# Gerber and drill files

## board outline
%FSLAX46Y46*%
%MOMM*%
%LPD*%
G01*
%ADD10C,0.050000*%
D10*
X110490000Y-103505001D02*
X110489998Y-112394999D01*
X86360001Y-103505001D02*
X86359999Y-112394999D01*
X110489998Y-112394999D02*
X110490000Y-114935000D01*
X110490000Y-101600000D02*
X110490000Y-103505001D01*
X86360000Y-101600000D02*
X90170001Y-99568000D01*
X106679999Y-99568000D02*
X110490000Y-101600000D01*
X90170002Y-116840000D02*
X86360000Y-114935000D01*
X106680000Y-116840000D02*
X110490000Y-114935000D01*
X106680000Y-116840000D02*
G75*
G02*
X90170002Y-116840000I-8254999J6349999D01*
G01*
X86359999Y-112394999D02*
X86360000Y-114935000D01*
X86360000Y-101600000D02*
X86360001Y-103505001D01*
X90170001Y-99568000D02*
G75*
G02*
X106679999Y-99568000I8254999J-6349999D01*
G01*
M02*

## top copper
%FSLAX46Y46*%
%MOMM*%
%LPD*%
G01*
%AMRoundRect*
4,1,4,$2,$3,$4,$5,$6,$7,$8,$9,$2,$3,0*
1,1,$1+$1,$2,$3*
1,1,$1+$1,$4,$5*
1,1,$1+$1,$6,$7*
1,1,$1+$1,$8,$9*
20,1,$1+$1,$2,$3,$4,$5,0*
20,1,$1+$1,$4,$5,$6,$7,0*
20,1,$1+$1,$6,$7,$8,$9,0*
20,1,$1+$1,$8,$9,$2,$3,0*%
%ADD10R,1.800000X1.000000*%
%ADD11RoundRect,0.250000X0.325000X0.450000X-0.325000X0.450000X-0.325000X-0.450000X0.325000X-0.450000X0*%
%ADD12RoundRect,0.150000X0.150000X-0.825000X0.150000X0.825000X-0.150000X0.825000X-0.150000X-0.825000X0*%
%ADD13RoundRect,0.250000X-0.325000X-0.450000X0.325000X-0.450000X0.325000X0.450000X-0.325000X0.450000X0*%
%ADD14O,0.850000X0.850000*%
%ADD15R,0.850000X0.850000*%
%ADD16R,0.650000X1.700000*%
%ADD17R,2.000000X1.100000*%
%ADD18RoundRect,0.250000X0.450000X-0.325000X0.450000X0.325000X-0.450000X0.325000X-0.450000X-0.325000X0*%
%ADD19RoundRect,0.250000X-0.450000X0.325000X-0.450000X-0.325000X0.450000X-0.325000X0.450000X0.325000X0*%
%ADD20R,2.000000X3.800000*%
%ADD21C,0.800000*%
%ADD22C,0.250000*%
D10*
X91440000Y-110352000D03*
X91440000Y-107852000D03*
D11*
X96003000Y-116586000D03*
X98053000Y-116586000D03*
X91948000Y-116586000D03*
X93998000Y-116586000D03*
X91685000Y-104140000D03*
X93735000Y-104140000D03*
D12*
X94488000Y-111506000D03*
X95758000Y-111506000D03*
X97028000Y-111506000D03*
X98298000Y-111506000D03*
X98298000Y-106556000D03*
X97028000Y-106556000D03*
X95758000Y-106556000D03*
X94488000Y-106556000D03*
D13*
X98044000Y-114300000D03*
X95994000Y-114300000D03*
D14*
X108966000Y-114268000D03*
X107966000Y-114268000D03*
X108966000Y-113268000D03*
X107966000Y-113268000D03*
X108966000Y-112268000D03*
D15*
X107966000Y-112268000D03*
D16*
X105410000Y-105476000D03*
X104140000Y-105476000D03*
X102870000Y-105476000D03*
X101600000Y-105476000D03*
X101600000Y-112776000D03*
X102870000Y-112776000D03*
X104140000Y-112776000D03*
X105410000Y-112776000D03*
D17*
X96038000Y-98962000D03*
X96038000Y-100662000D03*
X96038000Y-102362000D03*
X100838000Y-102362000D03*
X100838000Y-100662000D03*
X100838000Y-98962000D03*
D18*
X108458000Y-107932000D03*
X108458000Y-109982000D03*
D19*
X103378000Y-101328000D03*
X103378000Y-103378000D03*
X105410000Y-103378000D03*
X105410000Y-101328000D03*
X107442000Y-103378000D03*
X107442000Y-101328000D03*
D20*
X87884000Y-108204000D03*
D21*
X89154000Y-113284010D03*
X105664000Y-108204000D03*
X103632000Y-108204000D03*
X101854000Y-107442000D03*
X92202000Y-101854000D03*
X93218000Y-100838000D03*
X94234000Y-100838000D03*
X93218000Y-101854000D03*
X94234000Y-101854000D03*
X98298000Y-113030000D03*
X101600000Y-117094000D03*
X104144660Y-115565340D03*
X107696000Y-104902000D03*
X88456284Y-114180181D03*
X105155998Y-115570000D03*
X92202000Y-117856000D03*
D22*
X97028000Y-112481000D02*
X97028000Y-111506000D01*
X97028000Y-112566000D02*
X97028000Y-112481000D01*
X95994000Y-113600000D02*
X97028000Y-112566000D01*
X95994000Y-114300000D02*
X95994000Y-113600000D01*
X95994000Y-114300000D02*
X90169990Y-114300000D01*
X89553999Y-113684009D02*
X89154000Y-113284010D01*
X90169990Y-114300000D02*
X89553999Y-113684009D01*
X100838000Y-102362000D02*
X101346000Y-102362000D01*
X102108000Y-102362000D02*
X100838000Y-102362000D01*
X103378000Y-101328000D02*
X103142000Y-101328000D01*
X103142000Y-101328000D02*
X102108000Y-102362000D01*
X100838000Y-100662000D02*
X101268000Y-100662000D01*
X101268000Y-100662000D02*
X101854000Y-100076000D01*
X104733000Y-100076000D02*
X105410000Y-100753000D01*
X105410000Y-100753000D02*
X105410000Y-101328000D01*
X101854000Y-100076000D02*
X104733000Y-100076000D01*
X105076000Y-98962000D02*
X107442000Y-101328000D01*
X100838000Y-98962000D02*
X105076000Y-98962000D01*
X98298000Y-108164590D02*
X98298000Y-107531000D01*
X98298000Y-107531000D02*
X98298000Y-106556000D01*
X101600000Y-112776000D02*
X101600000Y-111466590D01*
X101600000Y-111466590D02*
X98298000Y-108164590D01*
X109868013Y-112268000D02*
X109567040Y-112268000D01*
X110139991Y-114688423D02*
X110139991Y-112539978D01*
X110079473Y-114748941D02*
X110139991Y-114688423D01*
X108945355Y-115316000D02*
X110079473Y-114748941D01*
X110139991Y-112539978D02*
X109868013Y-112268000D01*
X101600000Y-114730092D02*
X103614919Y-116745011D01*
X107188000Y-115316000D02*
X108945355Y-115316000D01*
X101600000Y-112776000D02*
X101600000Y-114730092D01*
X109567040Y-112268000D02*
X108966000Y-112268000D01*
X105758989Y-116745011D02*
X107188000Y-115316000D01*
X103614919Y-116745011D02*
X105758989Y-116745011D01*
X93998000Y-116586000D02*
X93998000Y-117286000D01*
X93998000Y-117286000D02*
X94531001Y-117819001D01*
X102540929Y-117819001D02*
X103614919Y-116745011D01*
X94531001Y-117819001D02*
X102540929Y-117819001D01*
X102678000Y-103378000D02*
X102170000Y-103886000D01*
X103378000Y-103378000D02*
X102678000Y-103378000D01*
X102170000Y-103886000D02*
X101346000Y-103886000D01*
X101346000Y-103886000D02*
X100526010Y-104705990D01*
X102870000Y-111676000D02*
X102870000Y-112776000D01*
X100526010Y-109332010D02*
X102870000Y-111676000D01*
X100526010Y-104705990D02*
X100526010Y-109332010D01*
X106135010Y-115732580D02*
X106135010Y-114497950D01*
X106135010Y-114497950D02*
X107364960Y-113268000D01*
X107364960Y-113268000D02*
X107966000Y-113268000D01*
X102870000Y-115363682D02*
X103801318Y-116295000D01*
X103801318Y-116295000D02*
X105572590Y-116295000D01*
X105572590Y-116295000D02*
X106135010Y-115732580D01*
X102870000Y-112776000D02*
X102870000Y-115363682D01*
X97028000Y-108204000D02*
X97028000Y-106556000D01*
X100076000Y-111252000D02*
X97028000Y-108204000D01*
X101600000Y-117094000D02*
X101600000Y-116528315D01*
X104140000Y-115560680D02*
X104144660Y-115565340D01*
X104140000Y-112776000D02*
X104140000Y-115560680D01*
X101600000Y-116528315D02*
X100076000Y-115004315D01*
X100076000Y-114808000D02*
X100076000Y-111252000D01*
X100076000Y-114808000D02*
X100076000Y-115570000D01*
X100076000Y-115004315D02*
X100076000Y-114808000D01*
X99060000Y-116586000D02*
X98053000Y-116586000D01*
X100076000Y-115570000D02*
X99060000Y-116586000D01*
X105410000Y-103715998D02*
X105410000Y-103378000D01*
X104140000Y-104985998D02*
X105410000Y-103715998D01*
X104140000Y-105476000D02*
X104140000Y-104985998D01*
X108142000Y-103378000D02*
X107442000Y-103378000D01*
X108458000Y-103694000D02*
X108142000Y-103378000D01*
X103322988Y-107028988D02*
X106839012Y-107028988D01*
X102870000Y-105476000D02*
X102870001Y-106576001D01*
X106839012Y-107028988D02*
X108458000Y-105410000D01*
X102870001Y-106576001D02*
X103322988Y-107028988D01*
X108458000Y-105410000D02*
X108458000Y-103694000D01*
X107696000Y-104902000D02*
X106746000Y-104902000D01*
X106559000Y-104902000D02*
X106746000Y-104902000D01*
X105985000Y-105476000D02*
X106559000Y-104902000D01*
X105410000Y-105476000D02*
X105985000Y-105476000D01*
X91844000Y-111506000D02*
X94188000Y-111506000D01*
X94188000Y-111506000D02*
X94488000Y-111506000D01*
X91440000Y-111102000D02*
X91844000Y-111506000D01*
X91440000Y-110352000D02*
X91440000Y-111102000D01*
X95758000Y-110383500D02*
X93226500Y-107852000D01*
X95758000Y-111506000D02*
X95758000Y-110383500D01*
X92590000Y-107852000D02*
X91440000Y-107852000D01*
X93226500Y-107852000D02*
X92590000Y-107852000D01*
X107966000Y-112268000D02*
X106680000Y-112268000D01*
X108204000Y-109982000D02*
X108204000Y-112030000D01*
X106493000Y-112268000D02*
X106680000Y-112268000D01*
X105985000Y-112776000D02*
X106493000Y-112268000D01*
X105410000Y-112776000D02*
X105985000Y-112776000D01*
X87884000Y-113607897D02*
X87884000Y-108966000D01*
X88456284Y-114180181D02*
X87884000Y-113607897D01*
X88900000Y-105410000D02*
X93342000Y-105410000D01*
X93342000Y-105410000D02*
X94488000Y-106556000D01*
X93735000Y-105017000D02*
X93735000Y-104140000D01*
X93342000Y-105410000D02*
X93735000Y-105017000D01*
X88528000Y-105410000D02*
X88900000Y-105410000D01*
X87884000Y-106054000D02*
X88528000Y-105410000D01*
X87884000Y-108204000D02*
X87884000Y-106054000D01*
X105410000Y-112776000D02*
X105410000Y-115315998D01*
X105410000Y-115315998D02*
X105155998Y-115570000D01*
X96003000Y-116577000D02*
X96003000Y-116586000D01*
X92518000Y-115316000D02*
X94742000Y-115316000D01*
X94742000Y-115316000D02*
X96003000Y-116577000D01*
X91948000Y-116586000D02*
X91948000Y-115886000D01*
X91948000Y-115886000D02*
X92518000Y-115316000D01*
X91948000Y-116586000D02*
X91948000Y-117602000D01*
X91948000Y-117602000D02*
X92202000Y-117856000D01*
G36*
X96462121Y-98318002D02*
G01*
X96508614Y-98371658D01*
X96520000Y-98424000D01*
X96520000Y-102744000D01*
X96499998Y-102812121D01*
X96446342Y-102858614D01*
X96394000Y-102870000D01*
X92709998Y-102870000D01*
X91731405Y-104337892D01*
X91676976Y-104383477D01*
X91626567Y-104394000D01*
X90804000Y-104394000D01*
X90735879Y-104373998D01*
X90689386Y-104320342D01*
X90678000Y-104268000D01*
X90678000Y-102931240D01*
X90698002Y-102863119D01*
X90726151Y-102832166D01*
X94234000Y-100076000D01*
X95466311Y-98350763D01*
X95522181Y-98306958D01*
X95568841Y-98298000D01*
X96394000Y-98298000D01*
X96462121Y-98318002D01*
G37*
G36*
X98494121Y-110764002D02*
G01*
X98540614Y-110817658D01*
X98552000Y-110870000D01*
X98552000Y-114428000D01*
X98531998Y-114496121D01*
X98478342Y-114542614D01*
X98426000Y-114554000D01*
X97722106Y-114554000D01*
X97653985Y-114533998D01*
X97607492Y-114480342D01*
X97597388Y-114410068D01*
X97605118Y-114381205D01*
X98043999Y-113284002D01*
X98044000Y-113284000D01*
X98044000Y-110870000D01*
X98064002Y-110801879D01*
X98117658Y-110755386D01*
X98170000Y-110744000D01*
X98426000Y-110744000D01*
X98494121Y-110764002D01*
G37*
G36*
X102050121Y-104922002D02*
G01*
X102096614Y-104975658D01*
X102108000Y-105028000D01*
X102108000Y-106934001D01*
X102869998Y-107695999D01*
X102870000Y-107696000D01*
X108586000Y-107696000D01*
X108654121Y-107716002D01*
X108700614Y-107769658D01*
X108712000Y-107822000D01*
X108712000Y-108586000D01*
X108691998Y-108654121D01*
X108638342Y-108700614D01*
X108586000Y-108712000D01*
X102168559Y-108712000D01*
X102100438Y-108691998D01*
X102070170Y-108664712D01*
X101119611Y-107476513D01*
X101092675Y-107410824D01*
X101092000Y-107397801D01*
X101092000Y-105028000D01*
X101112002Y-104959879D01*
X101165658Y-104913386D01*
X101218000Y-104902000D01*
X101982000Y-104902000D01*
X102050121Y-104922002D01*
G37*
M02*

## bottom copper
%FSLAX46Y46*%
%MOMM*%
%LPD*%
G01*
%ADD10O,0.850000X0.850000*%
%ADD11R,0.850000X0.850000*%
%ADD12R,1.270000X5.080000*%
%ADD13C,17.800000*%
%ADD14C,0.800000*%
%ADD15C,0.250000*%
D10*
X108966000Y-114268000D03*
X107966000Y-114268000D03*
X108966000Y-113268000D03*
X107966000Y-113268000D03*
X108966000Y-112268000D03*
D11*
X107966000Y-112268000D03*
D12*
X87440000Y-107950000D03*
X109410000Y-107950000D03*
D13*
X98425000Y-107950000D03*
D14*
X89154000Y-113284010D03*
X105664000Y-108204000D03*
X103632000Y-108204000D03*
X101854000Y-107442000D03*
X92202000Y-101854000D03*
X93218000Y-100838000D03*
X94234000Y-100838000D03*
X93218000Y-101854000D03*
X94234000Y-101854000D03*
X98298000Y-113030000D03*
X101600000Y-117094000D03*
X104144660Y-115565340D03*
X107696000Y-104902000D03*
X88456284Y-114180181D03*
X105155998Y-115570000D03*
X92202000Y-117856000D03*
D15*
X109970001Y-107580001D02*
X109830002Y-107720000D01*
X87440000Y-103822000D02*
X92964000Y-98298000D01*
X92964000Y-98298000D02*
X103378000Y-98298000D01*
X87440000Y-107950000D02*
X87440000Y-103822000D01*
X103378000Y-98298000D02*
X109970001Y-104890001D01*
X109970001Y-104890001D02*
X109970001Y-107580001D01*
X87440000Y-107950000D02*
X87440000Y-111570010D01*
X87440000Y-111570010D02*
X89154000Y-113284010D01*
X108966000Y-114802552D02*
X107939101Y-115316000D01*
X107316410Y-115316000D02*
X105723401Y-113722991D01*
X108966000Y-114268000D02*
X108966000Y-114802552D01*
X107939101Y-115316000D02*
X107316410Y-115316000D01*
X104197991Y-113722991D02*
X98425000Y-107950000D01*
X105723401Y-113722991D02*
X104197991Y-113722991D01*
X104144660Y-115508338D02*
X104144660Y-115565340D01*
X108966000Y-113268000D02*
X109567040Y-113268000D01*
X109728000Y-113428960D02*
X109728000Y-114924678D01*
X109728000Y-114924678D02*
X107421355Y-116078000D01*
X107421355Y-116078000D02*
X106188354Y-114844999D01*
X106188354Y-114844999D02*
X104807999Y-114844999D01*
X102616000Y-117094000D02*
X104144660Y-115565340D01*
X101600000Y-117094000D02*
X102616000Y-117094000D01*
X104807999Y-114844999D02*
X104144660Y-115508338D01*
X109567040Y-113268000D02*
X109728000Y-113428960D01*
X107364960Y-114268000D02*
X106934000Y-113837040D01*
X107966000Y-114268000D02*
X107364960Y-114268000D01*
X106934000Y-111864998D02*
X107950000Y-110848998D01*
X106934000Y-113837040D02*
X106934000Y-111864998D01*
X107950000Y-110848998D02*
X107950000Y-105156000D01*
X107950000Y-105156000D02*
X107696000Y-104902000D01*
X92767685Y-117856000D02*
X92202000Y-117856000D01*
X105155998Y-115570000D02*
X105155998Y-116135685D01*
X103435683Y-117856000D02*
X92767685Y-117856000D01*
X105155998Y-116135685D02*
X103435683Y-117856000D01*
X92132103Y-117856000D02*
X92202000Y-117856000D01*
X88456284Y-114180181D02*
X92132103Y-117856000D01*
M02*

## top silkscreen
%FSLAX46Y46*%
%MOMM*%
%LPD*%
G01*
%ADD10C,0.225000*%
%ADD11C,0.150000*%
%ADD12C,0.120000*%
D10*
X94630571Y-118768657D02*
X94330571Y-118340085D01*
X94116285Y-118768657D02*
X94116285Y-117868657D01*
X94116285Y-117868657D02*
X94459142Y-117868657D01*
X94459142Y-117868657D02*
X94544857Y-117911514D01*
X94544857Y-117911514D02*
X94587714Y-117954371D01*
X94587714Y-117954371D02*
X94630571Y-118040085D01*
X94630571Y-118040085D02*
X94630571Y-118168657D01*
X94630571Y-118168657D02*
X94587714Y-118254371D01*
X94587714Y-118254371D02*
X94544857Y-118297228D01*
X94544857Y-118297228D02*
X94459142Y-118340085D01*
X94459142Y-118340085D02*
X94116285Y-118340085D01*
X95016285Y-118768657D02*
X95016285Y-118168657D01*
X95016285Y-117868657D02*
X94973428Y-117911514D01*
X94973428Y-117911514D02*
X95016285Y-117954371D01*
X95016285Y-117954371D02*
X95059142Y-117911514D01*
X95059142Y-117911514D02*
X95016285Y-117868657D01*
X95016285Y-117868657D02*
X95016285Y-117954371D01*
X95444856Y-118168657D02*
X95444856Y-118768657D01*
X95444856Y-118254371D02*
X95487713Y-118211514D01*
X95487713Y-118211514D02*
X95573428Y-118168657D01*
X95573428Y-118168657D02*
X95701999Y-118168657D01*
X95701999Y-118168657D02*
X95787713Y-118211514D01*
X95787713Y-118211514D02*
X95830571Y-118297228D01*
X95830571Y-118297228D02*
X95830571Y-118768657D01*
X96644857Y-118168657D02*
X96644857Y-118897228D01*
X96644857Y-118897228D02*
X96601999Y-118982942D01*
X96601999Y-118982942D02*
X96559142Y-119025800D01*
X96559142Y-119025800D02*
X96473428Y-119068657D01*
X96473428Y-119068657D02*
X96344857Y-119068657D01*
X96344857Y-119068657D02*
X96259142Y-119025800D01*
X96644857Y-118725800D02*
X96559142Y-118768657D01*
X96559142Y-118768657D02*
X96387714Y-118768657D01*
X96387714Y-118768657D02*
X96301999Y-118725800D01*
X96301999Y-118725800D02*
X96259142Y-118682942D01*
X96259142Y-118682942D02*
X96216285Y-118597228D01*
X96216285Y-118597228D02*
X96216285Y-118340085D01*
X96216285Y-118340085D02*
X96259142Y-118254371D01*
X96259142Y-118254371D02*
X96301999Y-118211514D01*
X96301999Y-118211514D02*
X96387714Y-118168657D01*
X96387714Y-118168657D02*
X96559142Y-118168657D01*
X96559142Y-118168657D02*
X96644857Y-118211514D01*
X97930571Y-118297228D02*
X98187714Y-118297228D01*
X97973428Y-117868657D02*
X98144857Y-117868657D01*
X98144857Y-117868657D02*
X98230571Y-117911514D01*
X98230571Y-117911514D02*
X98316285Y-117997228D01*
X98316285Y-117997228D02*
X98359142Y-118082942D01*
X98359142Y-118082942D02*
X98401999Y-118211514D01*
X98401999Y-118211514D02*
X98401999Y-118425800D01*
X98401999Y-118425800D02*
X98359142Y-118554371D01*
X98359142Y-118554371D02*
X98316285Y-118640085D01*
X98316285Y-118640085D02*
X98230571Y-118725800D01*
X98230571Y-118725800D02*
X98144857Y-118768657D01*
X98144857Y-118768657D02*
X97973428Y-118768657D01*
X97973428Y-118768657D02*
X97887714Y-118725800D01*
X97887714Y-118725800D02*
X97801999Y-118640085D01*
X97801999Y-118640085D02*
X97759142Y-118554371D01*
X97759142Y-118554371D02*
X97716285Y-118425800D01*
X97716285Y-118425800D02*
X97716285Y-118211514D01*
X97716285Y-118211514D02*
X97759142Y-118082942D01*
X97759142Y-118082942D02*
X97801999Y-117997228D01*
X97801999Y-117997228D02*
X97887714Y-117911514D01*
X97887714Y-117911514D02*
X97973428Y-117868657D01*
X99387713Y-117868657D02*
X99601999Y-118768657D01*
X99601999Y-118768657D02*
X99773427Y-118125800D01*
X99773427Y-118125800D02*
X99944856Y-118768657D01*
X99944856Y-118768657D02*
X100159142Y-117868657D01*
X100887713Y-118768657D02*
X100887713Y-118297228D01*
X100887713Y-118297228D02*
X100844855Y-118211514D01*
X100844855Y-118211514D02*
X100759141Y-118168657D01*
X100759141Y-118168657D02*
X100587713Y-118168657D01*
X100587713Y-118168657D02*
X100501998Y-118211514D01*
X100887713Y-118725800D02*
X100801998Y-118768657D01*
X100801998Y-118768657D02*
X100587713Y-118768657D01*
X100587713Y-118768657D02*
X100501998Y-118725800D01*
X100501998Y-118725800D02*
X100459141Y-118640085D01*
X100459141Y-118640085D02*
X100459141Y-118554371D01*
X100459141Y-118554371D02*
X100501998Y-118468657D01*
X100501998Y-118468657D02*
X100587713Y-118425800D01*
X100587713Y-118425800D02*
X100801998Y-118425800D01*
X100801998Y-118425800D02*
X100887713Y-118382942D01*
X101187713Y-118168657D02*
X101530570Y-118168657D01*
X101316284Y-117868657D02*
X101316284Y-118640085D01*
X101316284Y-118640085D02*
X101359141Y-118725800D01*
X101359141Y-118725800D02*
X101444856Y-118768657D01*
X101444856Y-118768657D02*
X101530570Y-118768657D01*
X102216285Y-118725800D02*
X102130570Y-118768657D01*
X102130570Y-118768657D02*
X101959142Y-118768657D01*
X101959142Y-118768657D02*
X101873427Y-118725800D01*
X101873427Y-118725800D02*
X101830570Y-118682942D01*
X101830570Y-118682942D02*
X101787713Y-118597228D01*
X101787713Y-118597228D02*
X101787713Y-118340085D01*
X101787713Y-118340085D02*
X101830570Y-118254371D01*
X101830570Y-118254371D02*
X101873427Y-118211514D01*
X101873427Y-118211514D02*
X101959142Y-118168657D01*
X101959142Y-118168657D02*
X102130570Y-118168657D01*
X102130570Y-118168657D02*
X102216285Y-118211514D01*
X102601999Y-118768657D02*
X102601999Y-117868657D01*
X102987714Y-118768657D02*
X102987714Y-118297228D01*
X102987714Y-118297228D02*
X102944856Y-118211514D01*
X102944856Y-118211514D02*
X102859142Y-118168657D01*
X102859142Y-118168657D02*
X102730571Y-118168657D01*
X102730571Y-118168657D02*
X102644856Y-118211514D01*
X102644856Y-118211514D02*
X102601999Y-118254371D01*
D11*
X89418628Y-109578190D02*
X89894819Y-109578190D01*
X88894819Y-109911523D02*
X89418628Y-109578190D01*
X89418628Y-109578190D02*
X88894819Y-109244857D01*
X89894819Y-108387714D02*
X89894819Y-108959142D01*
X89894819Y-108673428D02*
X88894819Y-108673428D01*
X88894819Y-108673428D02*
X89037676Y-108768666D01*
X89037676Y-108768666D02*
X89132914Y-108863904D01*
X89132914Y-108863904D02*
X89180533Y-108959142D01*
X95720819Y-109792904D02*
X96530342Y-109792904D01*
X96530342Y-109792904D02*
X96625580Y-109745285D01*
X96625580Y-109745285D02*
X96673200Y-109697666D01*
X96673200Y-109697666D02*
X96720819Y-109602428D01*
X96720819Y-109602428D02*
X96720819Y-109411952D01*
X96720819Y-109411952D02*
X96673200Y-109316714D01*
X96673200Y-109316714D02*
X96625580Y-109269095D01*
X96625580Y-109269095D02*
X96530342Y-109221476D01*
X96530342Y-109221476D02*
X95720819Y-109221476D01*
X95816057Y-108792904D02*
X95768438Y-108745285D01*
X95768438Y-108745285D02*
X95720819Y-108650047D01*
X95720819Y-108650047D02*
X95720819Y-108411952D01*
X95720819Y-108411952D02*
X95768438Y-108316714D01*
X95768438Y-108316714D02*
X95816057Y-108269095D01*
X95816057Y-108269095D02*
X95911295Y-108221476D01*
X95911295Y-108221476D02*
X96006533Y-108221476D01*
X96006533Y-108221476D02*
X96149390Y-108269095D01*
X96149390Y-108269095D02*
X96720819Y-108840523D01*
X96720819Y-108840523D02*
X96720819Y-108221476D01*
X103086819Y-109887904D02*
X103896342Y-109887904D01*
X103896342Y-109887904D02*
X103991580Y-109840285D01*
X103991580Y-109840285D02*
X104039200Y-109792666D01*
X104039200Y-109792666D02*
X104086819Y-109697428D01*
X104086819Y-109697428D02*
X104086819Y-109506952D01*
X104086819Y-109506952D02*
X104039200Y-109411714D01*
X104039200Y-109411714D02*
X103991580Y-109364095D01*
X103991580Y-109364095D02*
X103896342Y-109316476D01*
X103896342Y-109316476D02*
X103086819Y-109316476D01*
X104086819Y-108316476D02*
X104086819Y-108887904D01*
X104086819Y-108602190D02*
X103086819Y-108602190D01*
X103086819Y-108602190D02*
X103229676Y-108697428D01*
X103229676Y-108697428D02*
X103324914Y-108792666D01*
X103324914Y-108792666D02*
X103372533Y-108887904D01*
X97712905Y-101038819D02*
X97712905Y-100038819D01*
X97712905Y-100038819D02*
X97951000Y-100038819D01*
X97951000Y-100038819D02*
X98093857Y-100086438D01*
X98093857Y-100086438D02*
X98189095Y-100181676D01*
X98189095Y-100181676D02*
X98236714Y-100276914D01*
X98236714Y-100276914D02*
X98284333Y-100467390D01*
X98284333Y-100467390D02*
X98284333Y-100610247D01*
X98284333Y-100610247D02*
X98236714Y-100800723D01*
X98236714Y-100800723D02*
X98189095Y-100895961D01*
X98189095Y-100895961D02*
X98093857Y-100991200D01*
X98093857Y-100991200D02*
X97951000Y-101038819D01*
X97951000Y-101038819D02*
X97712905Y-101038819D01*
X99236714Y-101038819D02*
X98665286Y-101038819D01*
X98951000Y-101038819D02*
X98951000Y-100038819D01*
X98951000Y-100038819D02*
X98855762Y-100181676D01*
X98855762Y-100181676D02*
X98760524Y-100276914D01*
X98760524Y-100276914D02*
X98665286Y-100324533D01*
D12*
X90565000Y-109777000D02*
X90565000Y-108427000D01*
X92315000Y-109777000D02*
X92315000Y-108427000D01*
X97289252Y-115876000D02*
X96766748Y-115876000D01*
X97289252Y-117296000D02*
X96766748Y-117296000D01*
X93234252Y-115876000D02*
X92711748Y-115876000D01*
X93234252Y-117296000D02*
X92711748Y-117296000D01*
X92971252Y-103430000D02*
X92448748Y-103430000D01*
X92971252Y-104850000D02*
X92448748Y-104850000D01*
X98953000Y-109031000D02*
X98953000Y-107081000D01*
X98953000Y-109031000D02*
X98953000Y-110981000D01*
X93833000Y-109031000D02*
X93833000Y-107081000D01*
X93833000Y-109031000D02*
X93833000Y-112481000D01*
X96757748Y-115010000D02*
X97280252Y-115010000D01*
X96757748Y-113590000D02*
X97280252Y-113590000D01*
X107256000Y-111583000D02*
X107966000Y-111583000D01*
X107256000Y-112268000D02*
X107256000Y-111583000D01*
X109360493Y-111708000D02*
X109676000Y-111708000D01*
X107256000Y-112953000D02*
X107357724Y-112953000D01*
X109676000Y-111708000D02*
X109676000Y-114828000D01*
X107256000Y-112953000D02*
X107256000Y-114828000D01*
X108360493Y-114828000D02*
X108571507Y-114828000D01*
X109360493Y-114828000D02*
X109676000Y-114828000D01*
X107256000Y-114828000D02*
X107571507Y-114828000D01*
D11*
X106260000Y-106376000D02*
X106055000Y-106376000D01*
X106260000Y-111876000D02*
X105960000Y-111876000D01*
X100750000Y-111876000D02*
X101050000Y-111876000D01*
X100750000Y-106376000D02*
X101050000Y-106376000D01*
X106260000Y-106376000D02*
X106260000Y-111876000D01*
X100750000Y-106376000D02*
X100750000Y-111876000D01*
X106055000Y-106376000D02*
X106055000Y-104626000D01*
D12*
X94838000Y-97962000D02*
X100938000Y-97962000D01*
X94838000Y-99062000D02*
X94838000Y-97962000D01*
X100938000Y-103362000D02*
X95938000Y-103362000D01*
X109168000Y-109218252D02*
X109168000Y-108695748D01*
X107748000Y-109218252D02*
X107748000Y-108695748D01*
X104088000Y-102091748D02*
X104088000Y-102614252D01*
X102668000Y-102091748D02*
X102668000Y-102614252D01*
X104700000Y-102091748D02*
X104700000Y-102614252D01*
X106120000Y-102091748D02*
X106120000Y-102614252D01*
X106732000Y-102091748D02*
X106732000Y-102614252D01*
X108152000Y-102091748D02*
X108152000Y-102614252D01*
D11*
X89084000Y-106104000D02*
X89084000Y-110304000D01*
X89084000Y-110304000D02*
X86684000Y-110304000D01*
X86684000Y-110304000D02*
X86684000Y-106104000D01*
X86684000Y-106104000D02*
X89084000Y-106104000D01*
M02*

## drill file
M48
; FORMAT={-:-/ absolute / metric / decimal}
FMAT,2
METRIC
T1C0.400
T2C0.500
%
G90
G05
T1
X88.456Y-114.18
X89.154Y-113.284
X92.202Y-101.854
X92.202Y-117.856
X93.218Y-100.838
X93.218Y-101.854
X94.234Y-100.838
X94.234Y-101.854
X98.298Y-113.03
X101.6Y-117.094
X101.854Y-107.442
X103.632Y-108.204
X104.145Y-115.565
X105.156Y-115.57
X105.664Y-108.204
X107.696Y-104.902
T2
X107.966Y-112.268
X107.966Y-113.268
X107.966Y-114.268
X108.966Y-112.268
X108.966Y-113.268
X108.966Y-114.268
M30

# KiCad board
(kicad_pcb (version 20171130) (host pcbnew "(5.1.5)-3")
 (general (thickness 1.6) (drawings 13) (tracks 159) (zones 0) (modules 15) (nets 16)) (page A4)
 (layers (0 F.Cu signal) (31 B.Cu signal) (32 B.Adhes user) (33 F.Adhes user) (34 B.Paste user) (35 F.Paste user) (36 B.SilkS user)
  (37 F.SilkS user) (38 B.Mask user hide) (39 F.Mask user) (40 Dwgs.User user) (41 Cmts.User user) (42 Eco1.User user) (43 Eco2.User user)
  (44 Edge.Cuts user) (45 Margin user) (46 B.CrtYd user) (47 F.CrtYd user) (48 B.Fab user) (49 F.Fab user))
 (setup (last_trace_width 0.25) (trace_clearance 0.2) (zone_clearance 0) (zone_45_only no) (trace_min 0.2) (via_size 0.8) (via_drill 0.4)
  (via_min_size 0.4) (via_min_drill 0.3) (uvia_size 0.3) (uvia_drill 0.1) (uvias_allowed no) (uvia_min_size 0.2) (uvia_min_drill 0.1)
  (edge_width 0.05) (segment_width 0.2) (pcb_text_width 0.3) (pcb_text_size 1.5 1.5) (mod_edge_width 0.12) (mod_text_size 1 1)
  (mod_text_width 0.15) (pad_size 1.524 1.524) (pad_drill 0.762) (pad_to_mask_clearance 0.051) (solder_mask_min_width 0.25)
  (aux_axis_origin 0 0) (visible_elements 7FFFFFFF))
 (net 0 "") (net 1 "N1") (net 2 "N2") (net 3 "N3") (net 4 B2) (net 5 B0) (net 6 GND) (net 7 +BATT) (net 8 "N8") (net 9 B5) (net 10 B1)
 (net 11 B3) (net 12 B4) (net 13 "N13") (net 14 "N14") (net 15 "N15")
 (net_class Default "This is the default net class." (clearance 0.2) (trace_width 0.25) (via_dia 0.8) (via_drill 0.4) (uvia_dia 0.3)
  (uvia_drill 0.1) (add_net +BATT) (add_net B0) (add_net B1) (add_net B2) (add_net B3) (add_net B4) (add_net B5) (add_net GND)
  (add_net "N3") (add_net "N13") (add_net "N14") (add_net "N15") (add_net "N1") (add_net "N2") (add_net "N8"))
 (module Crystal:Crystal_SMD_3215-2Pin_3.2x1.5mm (layer F.Cu) (at 91.44 109.102 90)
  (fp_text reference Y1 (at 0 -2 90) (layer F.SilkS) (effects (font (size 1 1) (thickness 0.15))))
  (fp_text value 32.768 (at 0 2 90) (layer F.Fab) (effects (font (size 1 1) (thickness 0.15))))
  (fp_line (start -0.675 -0.875) (end 0.675 -0.875) (layer F.SilkS) (width 0.12))
  (fp_line (start -0.675 0.875) (end 0.675 0.875) (layer F.SilkS) (width 0.12))
  (pad 2 smd rect (at -1.25 0 90) (size 1 1.8) (layers F.Cu F.Paste F.Mask) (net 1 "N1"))
  (pad 1 smd rect (at 1.25 0 90) (size 1 1.8) (layers F.Cu F.Paste F.Mask) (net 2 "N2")))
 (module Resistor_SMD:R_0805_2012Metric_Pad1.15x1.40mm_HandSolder (layer F.Cu) (at 97.028 116.586 180)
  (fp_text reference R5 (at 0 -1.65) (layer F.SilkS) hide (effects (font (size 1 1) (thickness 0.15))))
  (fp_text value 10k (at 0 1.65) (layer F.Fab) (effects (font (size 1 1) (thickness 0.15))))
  (fp_line (start -0.261252 0.71) (end 0.261252 0.71) (layer F.SilkS) (width 0.12))
  (fp_line (start -0.261252 -0.71) (end 0.261252 -0.71) (layer F.SilkS) (width 0.12))
  (pad 2 smd roundrect (at 1.025 0 180) (size 1.15 1.4) (layers F.Cu F.Paste F.Mask) (roundrect_rratio 0.217391) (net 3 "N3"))
  (pad 1 smd roundrect (at -1.025 0 180) (size 1.15 1.4) (layers F.Cu F.Paste F.Mask) (roundrect_rratio 0.217391) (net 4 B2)))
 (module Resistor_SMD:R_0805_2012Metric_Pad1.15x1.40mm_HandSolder (layer F.Cu) (at 92.973 116.586 180)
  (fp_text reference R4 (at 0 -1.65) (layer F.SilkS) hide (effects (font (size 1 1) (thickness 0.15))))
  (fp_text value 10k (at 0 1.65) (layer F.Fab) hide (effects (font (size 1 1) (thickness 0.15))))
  (fp_line (start -0.261252 0.71) (end 0.261252 0.71) (layer F.SilkS) (width 0.12))
  (fp_line (start -0.261252 -0.71) (end 0.261252 -0.71) (layer F.SilkS) (width 0.12))
  (pad 2 smd roundrect (at 1.025 0 180) (size 1.15 1.4) (layers F.Cu F.Paste F.Mask) (roundrect_rratio 0.217391) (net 3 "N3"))
  (pad 1 smd roundrect (at -1.025 0 180) (size 1.15 1.4) (layers F.Cu F.Paste F.Mask) (roundrect_rratio 0.217391) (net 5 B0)))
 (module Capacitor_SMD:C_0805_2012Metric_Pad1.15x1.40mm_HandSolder (layer F.Cu) (at 92.71 104.14 180)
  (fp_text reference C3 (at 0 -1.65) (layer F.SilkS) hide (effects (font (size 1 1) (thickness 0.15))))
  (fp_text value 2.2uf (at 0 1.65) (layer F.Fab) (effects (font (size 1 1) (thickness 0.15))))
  (fp_line (start -0.261252 0.71) (end 0.261252 0.71) (layer F.SilkS) (width 0.12))
  (fp_line (start -0.261252 -0.71) (end 0.261252 -0.71) (layer F.SilkS) (width 0.12))
  (pad 2 smd roundrect (at 1.025 0 180) (size 1.15 1.4) (layers F.Cu F.Paste F.Mask) (roundrect_rratio 0.217391) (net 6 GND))
  (pad 1 smd roundrect (at -1.025 0 180) (size 1.15 1.4) (layers F.Cu F.Paste F.Mask) (roundrect_rratio 0.217391) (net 3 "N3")))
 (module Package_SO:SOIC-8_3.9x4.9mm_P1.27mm (layer F.Cu) (at 96.393 109.031 90)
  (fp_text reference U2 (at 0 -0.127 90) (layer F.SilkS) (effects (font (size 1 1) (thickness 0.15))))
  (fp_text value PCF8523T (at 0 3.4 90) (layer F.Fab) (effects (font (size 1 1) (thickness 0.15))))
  (fp_line (start 0 2.56) (end 1.95 2.56) (layer F.SilkS) (width 0.12))
  (fp_line (start 0 2.56) (end -1.95 2.56) (layer F.SilkS) (width 0.12))
  (fp_line (start 0 -2.56) (end 1.95 -2.56) (layer F.SilkS) (width 0.12))
  (fp_line (start 0 -2.56) (end -3.45 -2.56) (layer F.SilkS) (width 0.12))
  (pad 1 smd roundrect (at -2.475 -1.905 90) (size 1.95 0.6) (layers F.Cu F.Paste F.Mask) (roundrect_rratio 0.25) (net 1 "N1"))
  (pad 2 smd roundrect (at -2.475 -0.635 90) (size 1.95 0.6) (layers F.Cu F.Paste F.Mask) (roundrect_rratio 0.25) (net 2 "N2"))
  (pad 3 smd roundrect (at -2.475 0.635 90) (size 1.95 0.6) (layers F.Cu F.Paste F.Mask) (roundrect_rratio 0.25) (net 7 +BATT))
  (pad 4 smd roundrect (at -2.475 1.905 90) (size 1.95 0.6) (layers F.Cu F.Paste F.Mask) (roundrect_rratio 0.25) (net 6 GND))
  (pad 5 smd roundrect (at 2.475 1.905 90) (size 1.95 0.6) (layers F.Cu F.Paste F.Mask) (roundrect_rratio 0.25) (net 5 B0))
  (pad 6 smd roundrect (at 2.475 0.635 90) (size 1.95 0.6) (layers F.Cu F.Paste F.Mask) (roundrect_rratio 0.25) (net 4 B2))
  (pad 7 smd roundrect (at 2.475 -0.635 90) (size 1.95 0.6) (layers F.Cu F.Paste F.Mask) (roundrect_rratio 0.25) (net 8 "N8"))
  (pad 8 smd roundrect (at 2.475 -1.905 90) (size 1.95 0.6) (layers F.Cu F.Paste F.Mask) (roundrect_rratio 0.25) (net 3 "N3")))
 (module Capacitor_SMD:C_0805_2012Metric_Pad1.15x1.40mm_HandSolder (layer F.Cu) (at 97.019 114.3)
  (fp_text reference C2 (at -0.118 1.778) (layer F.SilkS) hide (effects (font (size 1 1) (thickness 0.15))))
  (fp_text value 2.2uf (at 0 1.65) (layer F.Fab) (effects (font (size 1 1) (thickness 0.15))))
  (fp_line (start -0.261252 0.71) (end 0.261252 0.71) (layer F.SilkS) (width 0.12))
  (fp_line (start -0.261252 -0.71) (end 0.261252 -0.71) (layer F.SilkS) (width 0.12))
  (pad 2 smd roundrect (at 1.025 0) (size 1.15 1.4) (layers F.Cu F.Paste F.Mask) (roundrect_rratio 0.217391) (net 6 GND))
  (pad 1 smd roundrect (at -1.025 0) (size 1.15 1.4) (layers F.Cu F.Paste F.Mask) (roundrect_rratio 0.217391) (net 7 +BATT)))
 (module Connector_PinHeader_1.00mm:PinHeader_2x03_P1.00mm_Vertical (layer F.Cu) (at 107.966 112.268)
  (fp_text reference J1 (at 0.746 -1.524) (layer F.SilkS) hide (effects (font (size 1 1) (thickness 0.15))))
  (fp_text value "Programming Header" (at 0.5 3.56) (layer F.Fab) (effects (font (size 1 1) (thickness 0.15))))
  (fp_line (start -0.71 -0.685) (end 0 -0.685) (layer F.SilkS) (width 0.12))
  (fp_line (start -0.71 0) (end -0.71 -0.685) (layer F.SilkS) (width 0.12))
  (fp_line (start 1.394493 -0.56) (end 1.71 -0.56) (layer F.SilkS) (width 0.12))
  (fp_line (start -0.71 0.685) (end -0.608276 0.685) (layer F.SilkS) (width 0.12))
  (fp_line (start 1.71 -0.56) (end 1.71 2.56) (layer F.SilkS) (width 0.12))
  (fp_line (start -0.71 0.685) (end -0.71 2.56) (layer F.SilkS) (width 0.12))
  (fp_line (start 0.394493 2.56) (end 0.605507 2.56) (layer F.SilkS) (width 0.12))
  (fp_line (start 1.394493 2.56) (end 1.71 2.56) (layer F.SilkS) (width 0.12))
  (fp_line (start -0.71 2.56) (end -0.394493 2.56) (layer F.SilkS) (width 0.12))
  (pad 6 thru_hole oval (at 1 2) (size 0.85 0.85) (drill 0.5) (layers *.Cu *.Mask) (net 6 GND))
  (pad 5 thru_hole oval (at 0 2) (size 0.85 0.85) (drill 0.5) (layers *.Cu *.Mask) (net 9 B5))
  (pad 4 thru_hole oval (at 1 1) (size 0.85 0.85) (drill 0.5) (layers *.Cu *.Mask) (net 4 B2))
  (pad 3 thru_hole oval (at 0 1) (size 0.85 0.85) (drill 0.5) (layers *.Cu *.Mask) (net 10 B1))
  (pad 2 thru_hole oval (at 1 0) (size 0.85 0.85) (drill 0.5) (layers *.Cu *.Mask) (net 5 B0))
  (pad 1 thru_hole rect (at 0 0) (size 0.85 0.85) (drill 0.5) (layers *.Cu *.Mask) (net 3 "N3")))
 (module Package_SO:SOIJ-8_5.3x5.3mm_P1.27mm (layer F.Cu) (at 103.505 109.126 270)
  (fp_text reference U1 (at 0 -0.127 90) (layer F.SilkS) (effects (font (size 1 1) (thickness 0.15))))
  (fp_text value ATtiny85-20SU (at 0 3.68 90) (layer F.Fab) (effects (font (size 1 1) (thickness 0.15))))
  (fp_line (start -2.75 -2.755) (end -2.75 -2.55) (layer F.SilkS) (width 0.15))
  (fp_line (start 2.75 -2.755) (end 2.75 -2.455) (layer F.SilkS) (width 0.15))
  (fp_line (start 2.75 2.755) (end 2.75 2.455) (layer F.SilkS) (width 0.15))
  (fp_line (start -2.75 2.755) (end -2.75 2.455) (layer F.SilkS) (width 0.15))
  (fp_line (start -2.75 -2.755) (end 2.75 -2.755) (layer F.SilkS) (width 0.15))
  (fp_line (start -2.75 2.755) (end 2.75 2.755) (layer F.SilkS) (width 0.15))
  (fp_line (start -2.75 -2.55) (end -4.5 -2.55) (layer F.SilkS) (width 0.15))
  (pad 1 smd rect (at -3.65 -1.905 270) (size 1.7 0.65) (layers F.Cu F.Paste F.Mask) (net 9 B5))
  (pad 2 smd rect (at -3.65 -0.635 270) (size 1.7 0.65) (layers F.Cu F.Paste F.Mask) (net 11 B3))
  (pad 3 smd rect (at -3.65 0.635 270) (size 1.7 0.65) (layers F.Cu F.Paste F.Mask) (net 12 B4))
  (pad 4 smd rect (at -3.65 1.905 270) (size 1.7 0.65) (layers F.Cu F.Paste F.Mask) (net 6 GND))
  (pad 5 smd rect (at 3.65 1.905 270) (size 1.7 0.65) (layers F.Cu F.Paste F.Mask) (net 5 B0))
  (pad 6 smd rect (at 3.65 0.635 270) (size 1.7 0.65) (layers F.Cu F.Paste F.Mask) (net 10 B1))
  (pad 7 smd rect (at 3.65 -0.635 270) (size 1.7 0.65) (layers F.Cu F.Paste F.Mask) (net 4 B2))
  (pad 8 smd rect (at 3.65 -1.905 270) (size 1.7 0.65) (layers F.Cu F.Paste F.Mask) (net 3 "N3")))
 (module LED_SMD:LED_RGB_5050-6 (layer F.Cu) (at 98.438 100.662)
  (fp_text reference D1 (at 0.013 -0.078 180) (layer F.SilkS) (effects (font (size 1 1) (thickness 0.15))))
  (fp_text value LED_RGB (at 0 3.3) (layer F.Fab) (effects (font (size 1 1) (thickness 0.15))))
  (fp_line (start -3.6 -2.7) (end 2.5 -2.7) (layer F.SilkS) (width 0.12))
  (fp_line (start -3.6 -1.6) (end -3.6 -2.7) (layer F.SilkS) (width 0.12))
  (fp_line (start 2.5 2.7) (end -2.5 2.7) (layer F.SilkS) (width 0.12))
  (pad 1 smd rect (at -2.4 -1.7 90) (size 1.1 2) (layers F.Cu F.Paste F.Mask) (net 6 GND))
  (pad 2 smd rect (at -2.4 0 90) (size 1.1 2) (layers F.Cu F.Paste F.Mask) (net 6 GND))
  (pad 3 smd rect (at -2.4 1.7 90) (size 1.1 2) (layers F.Cu F.Paste F.Mask) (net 6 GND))
  (pad 4 smd rect (at 2.4 1.7 90) (size 1.1 2) (layers F.Cu F.Paste F.Mask) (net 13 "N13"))
  (pad 5 smd rect (at 2.4 0 90) (size 1.1 2) (layers F.Cu F.Paste F.Mask) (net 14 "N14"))
  (pad 6 smd rect (at 2.4 -1.7 90) (size 1.1 2) (layers F.Cu F.Paste F.Mask) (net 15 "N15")))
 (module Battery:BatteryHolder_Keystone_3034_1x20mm (layer B.Cu) (at 98.425 107.95)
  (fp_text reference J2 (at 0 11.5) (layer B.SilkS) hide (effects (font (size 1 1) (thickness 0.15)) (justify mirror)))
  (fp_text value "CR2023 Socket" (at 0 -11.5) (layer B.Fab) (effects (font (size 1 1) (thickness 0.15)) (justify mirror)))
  (pad 1 smd rect (at -10.985 0) (size 1.27 5.08) (layers B.Cu B.Paste B.Mask) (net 7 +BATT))
  (pad 1 smd rect (at 10.985 0) (size 1.27 5.08) (layers B.Cu B.Paste B.Mask) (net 7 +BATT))
  (pad 2 smd circle (at 0 0) (size 17.8 17.8) (layers B.Cu B.Mask) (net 6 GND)))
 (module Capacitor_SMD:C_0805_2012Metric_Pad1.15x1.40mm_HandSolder (layer F.Cu) (at 108.458 108.957 90)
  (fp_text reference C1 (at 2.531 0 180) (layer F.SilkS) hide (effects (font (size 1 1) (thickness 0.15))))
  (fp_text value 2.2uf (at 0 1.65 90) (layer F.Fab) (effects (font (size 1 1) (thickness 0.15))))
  (fp_line (start -0.261252 0.71) (end 0.261252 0.71) (layer F.SilkS) (width 0.12))
  (fp_line (start -0.261252 -0.71) (end 0.261252 -0.71) (layer F.SilkS) (width 0.12))
  (pad 2 smd roundrect (at 1.025 0 90) (size 1.15 1.4) (layers F.Cu F.Paste F.Mask) (roundrect_rratio 0.217391) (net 6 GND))
  (pad 1 smd roundrect (at -1.025 0 90) (size 1.15 1.4) (layers F.Cu F.Paste F.Mask) (roundrect_rratio 0.217391) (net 3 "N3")))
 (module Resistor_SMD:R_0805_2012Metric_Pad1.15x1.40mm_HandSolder (layer F.Cu) (at 103.378 102.353 270)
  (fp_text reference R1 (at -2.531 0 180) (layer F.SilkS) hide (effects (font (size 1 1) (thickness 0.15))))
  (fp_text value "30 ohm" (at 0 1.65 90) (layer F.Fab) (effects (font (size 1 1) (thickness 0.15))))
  (fp_line (start -0.261252 -0.71) (end 0.261252 -0.71) (layer F.SilkS) (width 0.12))
  (fp_line (start -0.261252 0.71) (end 0.261252 0.71) (layer F.SilkS) (width 0.12))
  (pad 1 smd roundrect (at -1.025 0 270) (size 1.15 1.4) (layers F.Cu F.Paste F.Mask) (roundrect_rratio 0.217391) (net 13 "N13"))
  (pad 2 smd roundrect (at 1.025 0 270) (size 1.15 1.4) (layers F.Cu F.Paste F.Mask) (roundrect_rratio 0.217391) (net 10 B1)))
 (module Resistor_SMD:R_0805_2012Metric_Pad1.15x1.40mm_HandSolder (layer F.Cu) (at 105.41 102.353 270)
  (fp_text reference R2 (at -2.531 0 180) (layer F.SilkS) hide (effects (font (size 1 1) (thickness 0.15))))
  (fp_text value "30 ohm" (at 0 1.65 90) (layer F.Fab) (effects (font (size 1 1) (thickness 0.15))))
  (fp_line (start -0.261252 0.71) (end 0.261252 0.71) (layer F.SilkS) (width 0.12))
  (fp_line (start -0.261252 -0.71) (end 0.261252 -0.71) (layer F.SilkS) (width 0.12))
  (pad 2 smd roundrect (at 1.025 0 270) (size 1.15 1.4) (layers F.Cu F.Paste F.Mask) (roundrect_rratio 0.217391) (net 11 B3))
  (pad 1 smd roundrect (at -1.025 0 270) (size 1.15 1.4) (layers F.Cu F.Paste F.Mask) (roundrect_rratio 0.217391) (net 14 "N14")))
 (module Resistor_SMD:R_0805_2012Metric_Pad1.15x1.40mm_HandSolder (layer F.Cu) (at 107.442 102.353 270)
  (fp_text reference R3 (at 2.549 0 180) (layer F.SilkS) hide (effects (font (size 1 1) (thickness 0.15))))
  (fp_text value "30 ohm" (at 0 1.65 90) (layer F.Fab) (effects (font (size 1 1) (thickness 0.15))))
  (fp_line (start -0.261252 0.71) (end 0.261252 0.71) (layer F.SilkS) (width 0.12))
  (fp_line (start -0.261252 -0.71) (end 0.261252 -0.71) (layer F.SilkS) (width 0.12))
  (pad 2 smd roundrect (at 1.025 0 270) (size 1.15 1.4) (layers F.Cu F.Paste F.Mask) (roundrect_rratio 0.217391) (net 12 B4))
  (pad 1 smd roundrect (at -1.025 0 270) (size 1.15 1.4) (layers F.Cu F.Paste F.Mask) (roundrect_rratio 0.217391) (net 15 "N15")))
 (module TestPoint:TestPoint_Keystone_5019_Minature (layer F.Cu) (at 87.884 108.204 270)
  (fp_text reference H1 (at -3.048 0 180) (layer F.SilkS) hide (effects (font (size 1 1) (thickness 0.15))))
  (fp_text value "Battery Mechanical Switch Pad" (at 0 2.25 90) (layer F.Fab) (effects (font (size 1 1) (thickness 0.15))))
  (fp_line (start -2.1 -1.2) (end 2.1 -1.2) (layer F.SilkS) (width 0.15))
  (fp_line (start 2.1 -1.2) (end 2.1 1.2) (layer F.SilkS) (width 0.15))
  (fp_line (start 2.1 1.2) (end -2.1 1.2) (layer F.SilkS) (width 0.15))
  (fp_line (start -2.1 1.2) (end -2.1 -1.2) (layer F.SilkS) (width 0.15))
  (pad 1 smd rect (at 0 0 270) (size 3.8 2) (layers F.Cu F.Paste F.Mask) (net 3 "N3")))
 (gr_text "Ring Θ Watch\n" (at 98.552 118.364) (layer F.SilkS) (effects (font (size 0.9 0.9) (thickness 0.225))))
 (gr_line (start 110.49 103.505001) (end 110.489998 112.394999) (layer Edge.Cuts) (width 0.05))
 (gr_line (start 86.360001 103.505001) (end 86.359999 112.394999) (layer Edge.Cuts) (width 0.05))
 (gr_line (start 110.489998 112.394999) (end 110.49 114.935) (layer Edge.Cuts) (width 0.05))
 (gr_line (start 110.49 101.6) (end 110.49 103.505001) (layer Edge.Cuts) (width 0.05))
 (gr_line (start 86.36 101.6) (end 90.170001 99.568) (layer Edge.Cuts) (width 0.05))
 (gr_line (start 106.679999 99.568) (end 110.49 101.6) (layer Edge.Cuts) (width 0.05))
 (gr_line (start 90.170002 116.84) (end 86.36 114.935) (layer Edge.Cuts) (width 0.05))
 (gr_line (start 106.68 116.84) (end 110.49 114.935) (layer Edge.Cuts) (width 0.05))
 (gr_arc (start 98.425001 110.490001) (end 90.170002 116.84) (angle -104.8628159) (layer Edge.Cuts) (width 0.05))
 (gr_line (start 86.359999 112.394999) (end 86.36 114.935) (layer Edge.Cuts) (width 0.05))
 (gr_line (start 86.36 101.6) (end 86.360001 103.505001) (layer Edge.Cuts) (width 0.05))
 (gr_arc (start 98.425 105.917999) (end 106.679999 99.568) (angle -104.8628159) (layer Edge.Cuts) (width 0.05))
 (segment (start 109.970001 107.580001) (end 109.830002 107.72) (width 0.25) (layer B.Cu) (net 7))
 (segment (start 87.44 103.822) (end 92.964 98.298) (width 0.25) (layer B.Cu) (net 7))
 (segment (start 92.964 98.298) (end 103.378 98.298) (width 0.25) (layer B.Cu) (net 7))
 (segment (start 87.44 107.95) (end 87.44 103.822) (width 0.25) (layer B.Cu) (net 7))
 (segment (start 103.378 98.298) (end 109.970001 104.890001) (width 0.25) (layer B.Cu) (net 7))
 (segment (start 109.970001 104.890001) (end 109.970001 107.580001) (width 0.25) (layer B.Cu) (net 7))
 (segment (start 97.028 112.481) (end 97.028 111.506) (width 0.25) (layer F.Cu) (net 7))
 (segment (start 97.028 112.566) (end 97.028 112.481) (width 0.25) (layer F.Cu) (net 7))
 (segment (start 95.994 113.6) (end 97.028 112.566) (width 0.25) (layer F.Cu) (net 7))
 (segment (start 95.994 114.3) (end 95.994 113.6) (width 0.25) (layer F.Cu) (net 7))
 (segment (start 87.44 107.95) (end 87.44 111.57001) (width 0.25) (layer B.Cu) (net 7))
 (segment (start 95.994 114.3) (end 90.16999 114.3) (width 0.25) (layer F.Cu) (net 7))
 (segment (start 87.44 111.57001) (end 89.154 113.28401) (width 0.25) (layer B.Cu) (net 7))
 (via (at 89.154 113.28401) (size 0.8) (drill 0.4) (layers F.Cu B.Cu) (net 7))
 (segment (start 89.553999 113.684009) (end 89.154 113.28401) (width 0.25) (layer F.Cu) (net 7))
 (segment (start 90.16999 114.3) (end 89.553999 113.684009) (width 0.25) (layer F.Cu) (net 7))
 (via (at 105.664 108.204) (size 0.8) (drill 0.4) (layers F.Cu B.Cu) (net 6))
 (via (at 103.632 108.204) (size 0.8) (drill 0.4) (layers F.Cu B.Cu) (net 6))
 (via (at 101.854 107.442) (size 0.8) (drill 0.4) (layers F.Cu B.Cu) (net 6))
 (via (at 92.202 101.854) (size 0.8) (drill 0.4) (layers F.Cu B.Cu) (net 6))
 (via (at 93.218 100.838) (size 0.8) (drill 0.4) (layers F.Cu B.Cu) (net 6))
 (via (at 94.234 100.838) (size 0.8) (drill 0.4) (layers F.Cu B.Cu) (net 6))
 (via (at 93.218 101.854) (size 0.8) (drill 0.4) (layers F.Cu B.Cu) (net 6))
 (via (at 94.234 101.854) (size 0.8) (drill 0.4) (layers F.Cu B.Cu) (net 6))
 (via (at 98.298 113.03) (size 0.8) (drill 0.4) (layers F.Cu B.Cu) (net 6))
 (segment (start 108.966 114.802552) (end 107.939101 115.316) (width 0.25) (layer B.Cu) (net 6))
 (segment (start 107.31641 115.316) (end 105.723401 113.722991) (width 0.25) (layer B.Cu) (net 6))
 (segment (start 108.966 114.268) (end 108.966 114.802552) (width 0.25) (layer B.Cu) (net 6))
 (segment (start 107.939101 115.316) (end 107.31641 115.316) (width 0.25) (layer B.Cu) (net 6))
 (segment (start 104.197991 113.722991) (end 98.425 107.95) (width 0.25) (layer B.Cu) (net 6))
 (segment (start 105.723401 113.722991) (end 104.197991 113.722991) (width 0.25) (layer B.Cu) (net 6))
 (segment (start 100.838 102.362) (end 101.346 102.362) (width 0.25) (layer F.Cu) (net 13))
 (segment (start 102.108 102.362) (end 100.838 102.362) (width 0.25) (layer F.Cu) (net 13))
 (segment (start 103.378 101.328) (end 103.142 101.328) (width 0.25) (layer F.Cu) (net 13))
 (segment (start 103.142 101.328) (end 102.108 102.362) (width 0.25) (layer F.Cu) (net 13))
 (segment (start 100.838 100.662) (end 101.268 100.662) (width 0.25) (layer F.Cu) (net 14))
 (segment (start 101.268 100.662) (end 101.854 100.076) (width 0.25) (layer F.Cu) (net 14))
 (segment (start 104.733 100.076) (end 105.41 100.753) (width 0.25) (layer F.Cu) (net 14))
 (segment (start 105.41 100.753) (end 105.41 101.328) (width 0.25) (layer F.Cu) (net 14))
 (segment (start 101.854 100.076) (end 104.733 100.076) (width 0.25) (layer F.Cu) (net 14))
 (segment (start 105.076 98.962) (end 107.442 101.328) (width 0.25) (layer F.Cu) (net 15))
 (segment (start 100.838 98.962) (end 105.076 98.962) (width 0.25) (layer F.Cu) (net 15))
 (segment (start 98.298 108.16459) (end 98.298 107.531) (width 0.25) (layer F.Cu) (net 5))
 (segment (start 98.298 107.531) (end 98.298 106.556) (width 0.25) (layer F.Cu) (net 5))
 (segment (start 101.6 112.776) (end 101.6 111.46659) (width 0.25) (layer F.Cu) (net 5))
 (segment (start 101.6 111.46659) (end 98.298 108.16459) (width 0.25) (layer F.Cu) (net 5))
 (segment (start 109.868013 112.268) (end 109.56704 112.268) (width 0.25) (layer F.Cu) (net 5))
 (segment (start 110.139991 114.688423) (end 110.139991 112.539978) (width 0.25) (layer F.Cu) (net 5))
 (segment (start 110.079473 114.748941) (end 110.139991 114.688423) (width 0.25) (layer F.Cu) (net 5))
 (segment (start 108.945355 115.316) (end 110.079473 114.748941) (width 0.25) (layer F.Cu) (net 5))
 (segment (start 110.139991 112.539978) (end 109.868013 112.268) (width 0.25) (layer F.Cu) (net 5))
 (segment (start 101.6 114.730092) (end 103.614919 116.745011) (width 0.25) (layer F.Cu) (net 5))
 (segment (start 107.188 115.316) (end 108.945355 115.316) (width 0.25) (layer F.Cu) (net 5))
 (segment (start 101.6 112.776) (end 101.6 114.730092) (width 0.25) (layer F.Cu) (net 5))
 (segment (start 109.56704 112.268) (end 108.966 112.268) (width 0.25) (layer F.Cu) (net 5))
 (segment (start 105.758989 116.745011) (end 107.188 115.316) (width 0.25) (layer F.Cu) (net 5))
 (segment (start 103.614919 116.745011) (end 105.758989 116.745011) (width 0.25) (layer F.Cu) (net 5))
 (segment (start 93.998 116.586) (end 93.998 117.286) (width 0.25) (layer F.Cu) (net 5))
 (segment (start 93.998 117.286) (end 94.531001 117.819001) (width 0.25) (layer F.Cu) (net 5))
 (segment (start 102.540929 117.819001) (end 103.614919 116.745011) (width 0.25) (layer F.Cu) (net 5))
 (segment (start 94.531001 117.819001) (end 102.540929 117.819001) (width 0.25) (layer F.Cu) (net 5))
 (segment (start 102.678 103.378) (end 102.17 103.886) (width 0.25) (layer F.Cu) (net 10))
 (segment (start 103.378 103.378) (end 102.678 103.378) (width 0.25) (layer F.Cu) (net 10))
 (segment (start 102.17 103.886) (end 101.346 103.886) (width 0.25) (layer F.Cu) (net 10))
 (segment (start 101.346 103.886) (end 100.52601 104.70599) (width 0.25) (layer F.Cu) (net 10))
 (segment (start 102.87 111.676) (end 102.87 112.776) (width 0.25) (layer F.Cu) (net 10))
 (segment (start 100.52601 109.33201) (end 102.87 111.676) (width 0.25) (layer F.Cu) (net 10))
 (segment (start 100.52601 104.70599) (end 100.52601 109.33201) (width 0.25) (layer F.Cu) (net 10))
 (segment (start 106.13501 115.73258) (end 106.13501 114.49795) (width 0.25) (layer F.Cu) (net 10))
 (segment (start 106.13501 114.49795) (end 107.36496 113.268) (width 0.25) (layer F.Cu) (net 10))
 (segment (start 107.36496 113.268) (end 107.966 113.268) (width 0.25) (layer F.Cu) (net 10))
 (segment (start 102.87 115.363682) (end 103.801318 116.295) (width 0.25) (layer F.Cu) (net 10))
 (segment (start 103.801318 116.295) (end 105.57259 116.295) (width 0.25) (layer F.Cu) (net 10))
 (segment (start 105.57259 116.295) (end 106.13501 115.73258) (width 0.25) (layer F.Cu) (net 10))
 (segment (start 102.87 112.776) (end 102.87 115.363682) (width 0.25) (layer F.Cu) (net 10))
 (via (at 101.6 117.094) (size 0.8) (drill 0.4) (layers F.Cu B.Cu) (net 4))
 (segment (start 97.028 108.204) (end 97.028 106.556) (width 0.25) (layer F.Cu) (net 4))
 (segment (start 100.076 111.252) (end 97.028 108.204) (width 0.25) (layer F.Cu) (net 4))
 (segment (start 101.6 117.094) (end 101.6 116.528315) (width 0.25) (layer F.Cu) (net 4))
 (via (at 104.14466 115.56534) (size 0.8) (drill 0.4) (layers F.Cu B.Cu) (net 4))
 (segment (start 104.14466 115.508338) (end 104.14466 115.56534) (width 0.25) (layer B.Cu) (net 4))
 (segment (start 108.966 113.268) (end 109.56704 113.268) (width 0.25) (layer B.Cu) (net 4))
 (segment (start 109.728 113.42896) (end 109.728 114.924678) (width 0.25) (layer B.Cu) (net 4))
 (segment (start 109.728 114.924678) (end 107.421355 116.078) (width 0.25) (layer B.Cu) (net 4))
 (segment (start 107.421355 116.078) (end 106.188354 114.844999) (width 0.25) (layer B.Cu) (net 4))
 (segment (start 106.188354 114.844999) (end 104.807999 114.844999) (width 0.25) (layer B.Cu) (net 4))
 (segment (start 102.616 117.094) (end 104.14466 115.56534) (width 0.25) (layer B.Cu) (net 4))
 (segment (start 104.14 115.56068) (end 104.14466 115.56534) (width 0.25) (layer F.Cu) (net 4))
 (segment (start 104.14 112.776) (end 104.14 115.56068) (width 0.25) (layer F.Cu) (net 4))
 (segment (start 101.6 117.094) (end 102.616 117.094) (width 0.25) (layer B.Cu) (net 4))
 (segment (start 104.807999 114.844999) (end 104.14466 115.508338) (width 0.25) (layer B.Cu) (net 4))
 (segment (start 109.56704 113.268) (end 109.728 113.42896) (width 0.25) (layer B.Cu) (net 4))
 (segment (start 101.6 116.528315) (end 100.076 115.004315) (width 0.25) (layer F.Cu) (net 4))
 (segment (start 100.076 114.808) (end 100.076 111.252) (width 0.25) (layer F.Cu) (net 4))
 (segment (start 100.076 114.808) (end 100.076 115.57) (width 0.25) (layer F.Cu) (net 4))
 (segment (start 100.076 115.004315) (end 100.076 114.808) (width 0.25) (layer F.Cu) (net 4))
 (segment (start 99.06 116.586) (end 98.053 116.586) (width 0.25) (layer F.Cu) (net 4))
 (segment (start 100.076 115.57) (end 99.06 116.586) (width 0.25) (layer F.Cu) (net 4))
 (segment (start 105.41 103.715998) (end 105.41 103.378) (width 0.25) (layer F.Cu) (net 11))
 (segment (start 104.14 104.985998) (end 105.41 103.715998) (width 0.25) (layer F.Cu) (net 11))
 (segment (start 104.14 105.476) (end 104.14 104.985998) (width 0.25) (layer F.Cu) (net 11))
 (segment (start 108.142 103.378) (end 107.442 103.378) (width 0.25) (layer F.Cu) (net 12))
 (segment (start 108.458 103.694) (end 108.142 103.378) (width 0.25) (layer F.Cu) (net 12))
 (segment (start 103.322988 107.028988) (end 106.839012 107.028988) (width 0.25) (layer F.Cu) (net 12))
 (segment (start 102.87 105.476) (end 102.870001 106.576001) (width 0.25) (layer F.Cu) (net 12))
 (segment (start 106.839012 107.028988) (end 108.458 105.41) (width 0.25) (layer F.Cu) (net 12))
 (segment (start 102.870001 106.576001) (end 103.322988 107.028988) (width 0.25) (layer F.Cu) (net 12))
 (segment (start 108.458 105.41) (end 108.458 103.694) (width 0.25) (layer F.Cu) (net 12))
 (segment (start 107.36496 114.268) (end 106.934 113.83704) (width 0.25) (layer B.Cu) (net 9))
 (segment (start 107.966 114.268) (end 107.36496 114.268) (width 0.25) (layer B.Cu) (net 9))
 (segment (start 106.934 111.864998) (end 107.95 110.848998) (width 0.25) (layer B.Cu) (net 9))
 (segment (start 106.934 113.83704) (end 106.934 111.864998) (width 0.25) (layer B.Cu) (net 9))
 (via (at 107.696 104.902) (size 0.8) (drill 0.4) (layers F.Cu B.Cu) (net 9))
 (segment (start 107.95 110.848998) (end 107.95 105.156) (width 0.25) (layer B.Cu) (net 9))
 (segment (start 107.95 105.156) (end 107.696 104.902) (width 0.25) (layer B.Cu) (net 9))
 (segment (start 107.696 104.902) (end 106.746 104.902) (width 0.25) (layer F.Cu) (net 9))
 (segment (start 106.559 104.902) (end 106.746 104.902) (width 0.25) (layer F.Cu) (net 9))
 (segment (start 105.985 105.476) (end 106.559 104.902) (width 0.25) (layer F.Cu) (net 9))
 (segment (start 105.41 105.476) (end 105.985 105.476) (width 0.25) (layer F.Cu) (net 9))
 (segment (start 91.844 111.506) (end 94.188 111.506) (width 0.25) (layer F.Cu) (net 1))
 (segment (start 94.188 111.506) (end 94.488 111.506) (width 0.25) (layer F.Cu) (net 1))
 (segment (start 91.44 111.102) (end 91.844 111.506) (width 0.25) (layer F.Cu) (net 1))
 (segment (start 91.44 110.352) (end 91.44 111.102) (width 0.25) (layer F.Cu) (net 1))
 (segment (start 95.758 110.3835) (end 93.2265 107.852) (width 0.25) (layer F.Cu) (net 2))
 (segment (start 95.758 111.506) (end 95.758 110.3835) (width 0.25) (layer F.Cu) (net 2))
 (segment (start 92.59 107.852) (end 91.44 107.852) (width 0.25) (layer F.Cu) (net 2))
 (segment (start 93.2265 107.852) (end 92.59 107.852) (width 0.25) (layer F.Cu) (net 2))
 (segment (start 107.966 112.268) (end 106.68 112.268) (width 0.25) (layer F.Cu) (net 3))
 (segment (start 108.204 109.982) (end 108.204 112.03) (width 0.25) (layer F.Cu) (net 3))
 (segment (start 106.493 112.268) (end 106.68 112.268) (width 0.25) (layer F.Cu) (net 3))
 (segment (start 105.985 112.776) (end 106.493 112.268) (width 0.25) (layer F.Cu) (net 3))
 (segment (start 105.41 112.776) (end 105.985 112.776) (width 0.25) (layer F.Cu) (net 3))
 (via (at 88.456284 114.180181) (size 0.8) (drill 0.4) (layers F.Cu B.Cu) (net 3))
 (segment (start 87.884 113.607897) (end 87.884 108.966) (width 0.25) (layer F.Cu) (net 3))
 (segment (start 88.456284 114.180181) (end 87.884 113.607897) (width 0.25) (layer F.Cu) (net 3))
 (segment (start 88.9 105.41) (end 93.342 105.41) (width 0.25) (layer F.Cu) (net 3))
 (segment (start 93.342 105.41) (end 94.488 106.556) (width 0.25) (layer F.Cu) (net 3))
 (segment (start 93.735 105.017) (end 93.735 104.14) (width 0.25) (layer F.Cu) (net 3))
 (segment (start 93.342 105.41) (end 93.735 105.017) (width 0.25) (layer F.Cu) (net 3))
 (segment (start 88.528 105.41) (end 88.9 105.41) (width 0.25) (layer F.Cu) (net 3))
 (segment (start 87.884 106.054) (end 88.528 105.41) (width 0.25) (layer F.Cu) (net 3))
 (segment (start 87.884 108.204) (end 87.884 106.054) (width 0.25) (layer F.Cu) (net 3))
 (via (at 105.155998 115.57) (size 0.8) (drill 0.4) (layers F.Cu B.Cu) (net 3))
 (segment (start 105.41 112.776) (end 105.41 115.315998) (width 0.25) (layer F.Cu) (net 3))
 (segment (start 105.41 115.315998) (end 105.155998 115.57) (width 0.25) (layer F.Cu) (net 3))
 (segment (start 96.003 116.577) (end 96.003 116.586) (width 0.25) (layer F.Cu) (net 3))
 (segment (start 92.518 115.316) (end 94.742 115.316) (width 0.25) (layer F.Cu) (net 3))
 (segment (start 94.742 115.316) (end 96.003 116.577) (width 0.25) (layer F.Cu) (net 3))
 (segment (start 91.948 116.586) (end 91.948 115.886) (width 0.25) (layer F.Cu) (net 3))
 (segment (start 91.948 115.886) (end 92.518 115.316) (width 0.25) (layer F.Cu) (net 3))
 (segment (start 92.767685 117.856) (end 92.202 117.856) (width 0.25) (layer B.Cu) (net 3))
 (via (at 92.202 117.856) (size 0.8) (drill 0.4) (layers F.Cu B.Cu) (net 3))
 (segment (start 91.948 116.586) (end 91.948 117.602) (width 0.25) (layer F.Cu) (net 3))
 (segment (start 105.155998 115.57) (end 105.155998 116.135685) (width 0.25) (layer B.Cu) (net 3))
 (segment (start 103.435683 117.856) (end 92.767685 117.856) (width 0.25) (layer B.Cu) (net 3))
 (segment (start 105.155998 116.135685) (end 103.435683 117.856) (width 0.25) (layer B.Cu) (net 3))
 (segment (start 92.132103 117.856) (end 92.202 117.856) (width 0.25) (layer B.Cu) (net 3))
 (segment (start 88.456284 114.180181) (end 92.132103 117.856) (width 0.25) (layer B.Cu) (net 3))
 (segment (start 91.948 117.602) (end 92.202 117.856) (width 0.25) (layer F.Cu) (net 3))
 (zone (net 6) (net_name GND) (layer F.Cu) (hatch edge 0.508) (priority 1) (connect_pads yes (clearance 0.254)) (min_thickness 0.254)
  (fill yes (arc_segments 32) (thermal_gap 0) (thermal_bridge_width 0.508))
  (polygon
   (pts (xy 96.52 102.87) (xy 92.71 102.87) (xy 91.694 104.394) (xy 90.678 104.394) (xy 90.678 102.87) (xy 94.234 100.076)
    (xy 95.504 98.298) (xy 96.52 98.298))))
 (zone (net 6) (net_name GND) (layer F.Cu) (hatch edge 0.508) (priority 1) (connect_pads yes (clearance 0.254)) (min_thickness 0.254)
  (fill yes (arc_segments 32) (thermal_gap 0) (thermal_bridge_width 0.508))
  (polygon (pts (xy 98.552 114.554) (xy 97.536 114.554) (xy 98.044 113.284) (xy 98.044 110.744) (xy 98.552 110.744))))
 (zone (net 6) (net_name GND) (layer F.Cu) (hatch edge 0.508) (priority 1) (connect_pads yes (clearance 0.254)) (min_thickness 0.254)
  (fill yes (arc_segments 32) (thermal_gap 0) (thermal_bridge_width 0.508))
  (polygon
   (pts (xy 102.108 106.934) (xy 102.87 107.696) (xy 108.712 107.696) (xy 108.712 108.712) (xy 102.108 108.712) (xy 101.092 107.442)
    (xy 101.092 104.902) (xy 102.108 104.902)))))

